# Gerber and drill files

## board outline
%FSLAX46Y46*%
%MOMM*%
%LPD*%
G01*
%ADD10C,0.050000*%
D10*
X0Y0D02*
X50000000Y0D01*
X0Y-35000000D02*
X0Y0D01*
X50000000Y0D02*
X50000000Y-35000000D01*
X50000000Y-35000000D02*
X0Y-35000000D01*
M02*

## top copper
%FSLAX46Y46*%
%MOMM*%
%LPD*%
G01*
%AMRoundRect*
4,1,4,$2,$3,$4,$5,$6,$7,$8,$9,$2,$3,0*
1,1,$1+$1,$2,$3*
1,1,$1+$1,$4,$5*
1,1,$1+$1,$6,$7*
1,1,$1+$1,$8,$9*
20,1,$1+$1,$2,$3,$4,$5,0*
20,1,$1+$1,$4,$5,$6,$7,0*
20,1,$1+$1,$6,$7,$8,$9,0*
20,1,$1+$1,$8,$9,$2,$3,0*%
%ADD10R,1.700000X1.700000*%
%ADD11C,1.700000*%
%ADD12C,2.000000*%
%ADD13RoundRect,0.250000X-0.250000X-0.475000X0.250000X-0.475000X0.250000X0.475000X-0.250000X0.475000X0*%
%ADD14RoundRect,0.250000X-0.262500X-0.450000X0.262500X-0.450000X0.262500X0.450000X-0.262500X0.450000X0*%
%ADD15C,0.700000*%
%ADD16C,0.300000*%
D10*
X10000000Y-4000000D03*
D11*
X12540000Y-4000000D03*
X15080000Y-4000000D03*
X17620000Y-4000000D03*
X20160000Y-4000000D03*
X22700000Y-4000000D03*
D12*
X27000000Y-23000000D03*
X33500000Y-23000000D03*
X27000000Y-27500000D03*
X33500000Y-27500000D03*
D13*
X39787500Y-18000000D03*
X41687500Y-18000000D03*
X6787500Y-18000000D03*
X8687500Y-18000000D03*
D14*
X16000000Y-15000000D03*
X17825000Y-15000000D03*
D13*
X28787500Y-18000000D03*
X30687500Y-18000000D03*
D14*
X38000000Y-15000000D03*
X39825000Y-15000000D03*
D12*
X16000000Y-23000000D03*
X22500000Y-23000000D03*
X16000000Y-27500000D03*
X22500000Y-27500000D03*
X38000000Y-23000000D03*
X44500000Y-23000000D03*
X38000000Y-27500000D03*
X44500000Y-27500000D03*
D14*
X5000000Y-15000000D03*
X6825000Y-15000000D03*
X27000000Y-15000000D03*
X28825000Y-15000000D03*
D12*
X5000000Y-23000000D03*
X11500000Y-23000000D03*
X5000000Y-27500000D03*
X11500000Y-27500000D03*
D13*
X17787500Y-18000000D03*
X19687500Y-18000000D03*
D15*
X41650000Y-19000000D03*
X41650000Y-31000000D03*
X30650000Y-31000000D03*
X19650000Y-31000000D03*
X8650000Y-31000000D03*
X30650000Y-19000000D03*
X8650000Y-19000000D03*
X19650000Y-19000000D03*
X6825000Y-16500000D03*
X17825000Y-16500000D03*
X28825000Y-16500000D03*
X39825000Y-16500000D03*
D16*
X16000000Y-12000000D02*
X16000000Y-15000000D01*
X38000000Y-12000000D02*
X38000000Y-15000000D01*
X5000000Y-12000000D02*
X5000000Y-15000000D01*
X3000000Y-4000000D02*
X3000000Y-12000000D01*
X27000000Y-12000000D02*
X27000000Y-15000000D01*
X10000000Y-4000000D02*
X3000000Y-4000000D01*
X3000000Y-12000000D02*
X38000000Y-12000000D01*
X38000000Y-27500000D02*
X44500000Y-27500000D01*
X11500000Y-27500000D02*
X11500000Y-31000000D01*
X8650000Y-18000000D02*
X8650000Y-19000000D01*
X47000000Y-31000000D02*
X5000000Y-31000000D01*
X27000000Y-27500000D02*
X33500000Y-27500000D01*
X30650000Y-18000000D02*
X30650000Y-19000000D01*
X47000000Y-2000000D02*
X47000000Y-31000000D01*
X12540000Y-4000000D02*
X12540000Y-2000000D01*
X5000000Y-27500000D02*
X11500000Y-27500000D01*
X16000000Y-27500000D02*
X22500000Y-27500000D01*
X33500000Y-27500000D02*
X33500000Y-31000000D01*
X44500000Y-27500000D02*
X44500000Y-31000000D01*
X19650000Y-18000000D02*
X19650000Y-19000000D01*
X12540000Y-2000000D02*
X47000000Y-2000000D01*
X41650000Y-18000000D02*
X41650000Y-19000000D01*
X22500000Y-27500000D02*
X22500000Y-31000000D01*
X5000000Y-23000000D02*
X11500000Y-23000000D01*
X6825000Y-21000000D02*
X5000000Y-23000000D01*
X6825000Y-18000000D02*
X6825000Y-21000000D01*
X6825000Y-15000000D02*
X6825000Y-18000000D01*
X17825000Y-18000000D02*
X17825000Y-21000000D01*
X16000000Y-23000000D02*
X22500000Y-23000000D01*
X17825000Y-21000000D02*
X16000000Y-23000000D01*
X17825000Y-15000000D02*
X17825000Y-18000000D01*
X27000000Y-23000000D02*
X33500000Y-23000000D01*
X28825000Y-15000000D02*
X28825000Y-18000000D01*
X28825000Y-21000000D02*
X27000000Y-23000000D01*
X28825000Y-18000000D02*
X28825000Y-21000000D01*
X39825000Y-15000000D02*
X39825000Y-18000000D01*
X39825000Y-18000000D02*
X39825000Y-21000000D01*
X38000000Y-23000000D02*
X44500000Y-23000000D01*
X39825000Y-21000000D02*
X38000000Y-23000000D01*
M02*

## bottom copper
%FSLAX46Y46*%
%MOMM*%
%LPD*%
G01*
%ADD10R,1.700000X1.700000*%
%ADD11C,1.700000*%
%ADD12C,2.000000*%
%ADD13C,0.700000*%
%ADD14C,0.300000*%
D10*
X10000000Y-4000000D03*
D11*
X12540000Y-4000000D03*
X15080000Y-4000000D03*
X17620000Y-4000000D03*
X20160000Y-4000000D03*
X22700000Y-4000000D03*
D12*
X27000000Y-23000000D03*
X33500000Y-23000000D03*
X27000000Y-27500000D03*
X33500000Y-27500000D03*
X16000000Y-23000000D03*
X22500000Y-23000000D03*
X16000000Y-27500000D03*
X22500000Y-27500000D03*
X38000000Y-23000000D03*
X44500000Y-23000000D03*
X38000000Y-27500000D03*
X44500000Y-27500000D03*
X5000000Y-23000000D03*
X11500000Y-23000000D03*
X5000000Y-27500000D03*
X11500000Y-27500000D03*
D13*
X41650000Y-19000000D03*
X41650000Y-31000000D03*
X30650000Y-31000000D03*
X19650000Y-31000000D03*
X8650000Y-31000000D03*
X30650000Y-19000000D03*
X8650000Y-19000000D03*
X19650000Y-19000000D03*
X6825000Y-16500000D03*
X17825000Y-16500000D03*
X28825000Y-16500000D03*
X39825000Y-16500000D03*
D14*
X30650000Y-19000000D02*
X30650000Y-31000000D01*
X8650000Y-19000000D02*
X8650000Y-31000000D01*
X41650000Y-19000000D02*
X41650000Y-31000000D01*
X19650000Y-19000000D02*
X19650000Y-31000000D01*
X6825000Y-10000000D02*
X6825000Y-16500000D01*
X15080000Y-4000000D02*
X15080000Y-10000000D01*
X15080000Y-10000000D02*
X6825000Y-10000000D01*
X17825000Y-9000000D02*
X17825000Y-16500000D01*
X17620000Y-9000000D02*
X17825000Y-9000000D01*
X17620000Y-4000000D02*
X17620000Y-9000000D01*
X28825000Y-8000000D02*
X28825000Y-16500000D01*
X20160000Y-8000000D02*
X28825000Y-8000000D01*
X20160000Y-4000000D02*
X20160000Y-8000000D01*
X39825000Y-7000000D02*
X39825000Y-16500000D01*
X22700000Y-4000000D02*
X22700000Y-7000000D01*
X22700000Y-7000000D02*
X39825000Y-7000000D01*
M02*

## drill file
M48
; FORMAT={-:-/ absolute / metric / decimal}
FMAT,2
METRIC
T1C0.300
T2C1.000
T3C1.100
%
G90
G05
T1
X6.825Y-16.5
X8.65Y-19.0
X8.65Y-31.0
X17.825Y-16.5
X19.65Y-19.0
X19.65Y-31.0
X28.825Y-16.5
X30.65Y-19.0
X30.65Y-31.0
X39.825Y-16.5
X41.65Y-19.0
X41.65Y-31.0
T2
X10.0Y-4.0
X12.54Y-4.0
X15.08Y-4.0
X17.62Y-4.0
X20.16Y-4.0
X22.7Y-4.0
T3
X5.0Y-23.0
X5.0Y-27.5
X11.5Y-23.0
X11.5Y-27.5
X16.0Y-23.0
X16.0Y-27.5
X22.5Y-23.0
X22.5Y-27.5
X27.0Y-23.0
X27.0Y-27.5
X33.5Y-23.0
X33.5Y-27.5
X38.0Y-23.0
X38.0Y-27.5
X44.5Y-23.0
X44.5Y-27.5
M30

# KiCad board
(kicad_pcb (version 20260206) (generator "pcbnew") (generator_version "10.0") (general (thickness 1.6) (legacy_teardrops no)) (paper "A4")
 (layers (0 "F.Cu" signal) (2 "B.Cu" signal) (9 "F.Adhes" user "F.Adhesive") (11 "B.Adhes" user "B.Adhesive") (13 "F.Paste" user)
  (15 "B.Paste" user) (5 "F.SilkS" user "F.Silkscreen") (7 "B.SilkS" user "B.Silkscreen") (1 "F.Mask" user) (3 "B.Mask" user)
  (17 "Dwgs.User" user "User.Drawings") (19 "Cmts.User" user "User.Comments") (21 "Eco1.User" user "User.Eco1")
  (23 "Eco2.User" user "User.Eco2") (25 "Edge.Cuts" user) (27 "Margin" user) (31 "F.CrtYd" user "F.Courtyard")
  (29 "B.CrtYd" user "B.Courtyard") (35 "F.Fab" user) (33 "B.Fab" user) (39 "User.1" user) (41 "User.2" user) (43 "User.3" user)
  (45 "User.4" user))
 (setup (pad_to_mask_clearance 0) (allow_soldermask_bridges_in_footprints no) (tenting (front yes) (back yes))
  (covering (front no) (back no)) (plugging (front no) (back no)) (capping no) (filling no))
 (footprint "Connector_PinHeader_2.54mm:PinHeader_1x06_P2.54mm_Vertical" (layer "F.Cu") (at 10 4 90)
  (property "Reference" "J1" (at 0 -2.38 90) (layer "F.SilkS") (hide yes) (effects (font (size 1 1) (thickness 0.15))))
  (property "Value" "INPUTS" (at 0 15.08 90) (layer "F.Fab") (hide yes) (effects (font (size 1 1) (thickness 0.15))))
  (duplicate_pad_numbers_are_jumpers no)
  (pad "1" thru_hole rect (at 0 0 90) (size 1.7 1.7) (drill 1) (layers "*.Cu" "*.Mask") (remove_unused_layers no) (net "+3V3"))
  (pad "2" thru_hole circle (at 0 2.54 90) (size 1.7 1.7) (drill 1) (layers "*.Cu" "*.Mask") (remove_unused_layers no) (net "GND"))
  (pad "3" thru_hole circle (at 0 5.08 90) (size 1.7 1.7) (drill 1) (layers "*.Cu" "*.Mask") (remove_unused_layers no) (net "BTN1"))
  (pad "4" thru_hole circle (at 0 7.62 90) (size 1.7 1.7) (drill 1) (layers "*.Cu" "*.Mask") (remove_unused_layers no) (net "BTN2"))
  (pad "5" thru_hole circle (at 0 10.16 90) (size 1.7 1.7) (drill 1) (layers "*.Cu" "*.Mask") (remove_unused_layers no) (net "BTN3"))
  (pad "6" thru_hole circle (at 0 12.7 90) (size 1.7 1.7) (drill 1) (layers "*.Cu" "*.Mask") (remove_unused_layers no) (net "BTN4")))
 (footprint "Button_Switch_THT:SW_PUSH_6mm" (layer "F.Cu") (at 27 23)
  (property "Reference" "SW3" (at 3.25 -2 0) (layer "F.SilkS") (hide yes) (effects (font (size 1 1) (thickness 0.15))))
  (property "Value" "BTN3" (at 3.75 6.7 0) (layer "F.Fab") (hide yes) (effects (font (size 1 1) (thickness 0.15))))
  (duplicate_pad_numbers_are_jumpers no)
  (pad "1" thru_hole circle (at 0 0 90) (size 2 2) (drill 1.1) (layers "*.Cu" "*.Mask") (remove_unused_layers no) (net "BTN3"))
  (pad "1" thru_hole circle (at 6.5 0 90) (size 2 2) (drill 1.1) (layers "*.Cu" "*.Mask") (remove_unused_layers no) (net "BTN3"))
  (pad "2" thru_hole circle (at 0 4.5 90) (size 2 2) (drill 1.1) (layers "*.Cu" "*.Mask") (remove_unused_layers no) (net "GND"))
  (pad "2" thru_hole circle (at 6.5 4.5 90) (size 2 2) (drill 1.1) (layers "*.Cu" "*.Mask") (remove_unused_layers no) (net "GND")))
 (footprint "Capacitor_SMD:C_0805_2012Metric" (layer "F.Cu") (at 40.7375 18)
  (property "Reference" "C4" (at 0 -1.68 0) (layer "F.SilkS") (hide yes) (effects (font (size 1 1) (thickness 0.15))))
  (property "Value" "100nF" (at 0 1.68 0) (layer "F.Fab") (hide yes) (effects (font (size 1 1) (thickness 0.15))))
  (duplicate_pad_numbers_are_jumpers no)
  (pad "1" smd roundrect (at -0.95 0) (size 1 1.45) (layers "F.Cu" "F.Mask" "F.Paste") (roundrect_rratio 0.25) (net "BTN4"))
  (pad "2" smd roundrect (at 0.95 0) (size 1 1.45) (layers "F.Cu" "F.Mask" "F.Paste") (roundrect_rratio 0.25) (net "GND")))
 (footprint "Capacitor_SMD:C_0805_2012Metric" (layer "F.Cu") (at 7.7375 18)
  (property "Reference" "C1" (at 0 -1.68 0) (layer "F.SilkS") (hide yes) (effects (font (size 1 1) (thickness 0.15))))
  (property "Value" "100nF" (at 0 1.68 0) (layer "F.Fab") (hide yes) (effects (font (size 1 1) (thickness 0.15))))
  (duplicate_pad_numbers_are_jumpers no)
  (pad "1" smd roundrect (at -0.95 0) (size 1 1.45) (layers "F.Cu" "F.Mask" "F.Paste") (roundrect_rratio 0.25) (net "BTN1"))
  (pad "2" smd roundrect (at 0.95 0) (size 1 1.45) (layers "F.Cu" "F.Mask" "F.Paste") (roundrect_rratio 0.25) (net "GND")))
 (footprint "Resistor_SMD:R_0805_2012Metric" (layer "F.Cu") (at 16.9125 15)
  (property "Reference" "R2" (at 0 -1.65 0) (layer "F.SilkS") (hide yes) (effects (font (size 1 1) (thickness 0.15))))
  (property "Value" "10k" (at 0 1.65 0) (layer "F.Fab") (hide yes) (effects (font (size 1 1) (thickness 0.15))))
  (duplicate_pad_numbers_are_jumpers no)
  (pad "1" smd roundrect (at -0.9125 0) (size 1.025 1.4) (layers "F.Cu" "F.Mask" "F.Paste") (roundrect_rratio 0.243902) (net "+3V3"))
  (pad "2" smd roundrect (at 0.9125 0) (size 1.025 1.4) (layers "F.Cu" "F.Mask" "F.Paste") (roundrect_rratio 0.243902) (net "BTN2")))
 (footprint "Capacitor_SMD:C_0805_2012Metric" (layer "F.Cu") (at 29.7375 18)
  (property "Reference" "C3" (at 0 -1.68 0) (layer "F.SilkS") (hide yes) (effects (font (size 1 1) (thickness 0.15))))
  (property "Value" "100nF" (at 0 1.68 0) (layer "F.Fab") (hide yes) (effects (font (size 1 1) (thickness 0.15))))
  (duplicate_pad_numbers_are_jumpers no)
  (pad "1" smd roundrect (at -0.95 0) (size 1 1.45) (layers "F.Cu" "F.Mask" "F.Paste") (roundrect_rratio 0.25) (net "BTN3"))
  (pad "2" smd roundrect (at 0.95 0) (size 1 1.45) (layers "F.Cu" "F.Mask" "F.Paste") (roundrect_rratio 0.25) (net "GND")))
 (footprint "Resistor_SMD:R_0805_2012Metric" (layer "F.Cu") (at 38.9125 15)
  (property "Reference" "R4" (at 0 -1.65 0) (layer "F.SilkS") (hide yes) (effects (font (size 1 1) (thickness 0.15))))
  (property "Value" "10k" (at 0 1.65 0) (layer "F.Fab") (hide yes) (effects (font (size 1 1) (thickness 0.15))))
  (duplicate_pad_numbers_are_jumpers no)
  (pad "1" smd roundrect (at -0.9125 0) (size 1.025 1.4) (layers "F.Cu" "F.Mask" "F.Paste") (roundrect_rratio 0.243902) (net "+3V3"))
  (pad "2" smd roundrect (at 0.9125 0) (size 1.025 1.4) (layers "F.Cu" "F.Mask" "F.Paste") (roundrect_rratio 0.243902) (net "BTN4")))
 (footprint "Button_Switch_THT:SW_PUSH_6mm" (layer "F.Cu") (at 16 23)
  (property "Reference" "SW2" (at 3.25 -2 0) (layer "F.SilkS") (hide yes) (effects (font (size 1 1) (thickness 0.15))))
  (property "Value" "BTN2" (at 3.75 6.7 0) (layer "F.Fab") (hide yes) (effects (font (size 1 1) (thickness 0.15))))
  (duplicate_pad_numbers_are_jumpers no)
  (pad "1" thru_hole circle (at 0 0 90) (size 2 2) (drill 1.1) (layers "*.Cu" "*.Mask") (remove_unused_layers no) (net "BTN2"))
  (pad "1" thru_hole circle (at 6.5 0 90) (size 2 2) (drill 1.1) (layers "*.Cu" "*.Mask") (remove_unused_layers no) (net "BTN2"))
  (pad "2" thru_hole circle (at 0 4.5 90) (size 2 2) (drill 1.1) (layers "*.Cu" "*.Mask") (remove_unused_layers no) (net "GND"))
  (pad "2" thru_hole circle (at 6.5 4.5 90) (size 2 2) (drill 1.1) (layers "*.Cu" "*.Mask") (remove_unused_layers no) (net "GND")))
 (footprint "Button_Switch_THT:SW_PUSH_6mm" (layer "F.Cu") (at 38 23)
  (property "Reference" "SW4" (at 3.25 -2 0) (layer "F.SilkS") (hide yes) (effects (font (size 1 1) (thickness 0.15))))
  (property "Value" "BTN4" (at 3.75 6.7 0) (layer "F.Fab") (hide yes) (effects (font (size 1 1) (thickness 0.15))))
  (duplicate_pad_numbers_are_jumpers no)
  (pad "1" thru_hole circle (at 0 0 90) (size 2 2) (drill 1.1) (layers "*.Cu" "*.Mask") (remove_unused_layers no) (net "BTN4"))
  (pad "1" thru_hole circle (at 6.5 0 90) (size 2 2) (drill 1.1) (layers "*.Cu" "*.Mask") (remove_unused_layers no) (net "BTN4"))
  (pad "2" thru_hole circle (at 0 4.5 90) (size 2 2) (drill 1.1) (layers "*.Cu" "*.Mask") (remove_unused_layers no) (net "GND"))
  (pad "2" thru_hole circle (at 6.5 4.5 90) (size 2 2) (drill 1.1) (layers "*.Cu" "*.Mask") (remove_unused_layers no) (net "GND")))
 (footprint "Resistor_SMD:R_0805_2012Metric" (layer "F.Cu") (at 5.9125 15)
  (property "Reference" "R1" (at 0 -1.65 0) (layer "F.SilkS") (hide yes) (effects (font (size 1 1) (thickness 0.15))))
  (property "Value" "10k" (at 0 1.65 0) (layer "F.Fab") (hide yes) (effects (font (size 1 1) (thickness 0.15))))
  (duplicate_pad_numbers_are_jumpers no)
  (pad "1" smd roundrect (at -0.9125 0) (size 1.025 1.4) (layers "F.Cu" "F.Mask" "F.Paste") (roundrect_rratio 0.243902) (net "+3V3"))
  (pad "2" smd roundrect (at 0.9125 0) (size 1.025 1.4) (layers "F.Cu" "F.Mask" "F.Paste") (roundrect_rratio 0.243902) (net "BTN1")))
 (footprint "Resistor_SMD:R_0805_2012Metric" (layer "F.Cu") (at 27.9125 15)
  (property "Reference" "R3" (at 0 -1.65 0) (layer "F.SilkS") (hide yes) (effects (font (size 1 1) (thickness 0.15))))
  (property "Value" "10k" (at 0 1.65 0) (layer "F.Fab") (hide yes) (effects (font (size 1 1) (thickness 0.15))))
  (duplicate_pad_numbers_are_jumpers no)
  (pad "1" smd roundrect (at -0.9125 0) (size 1.025 1.4) (layers "F.Cu" "F.Mask" "F.Paste") (roundrect_rratio 0.243902) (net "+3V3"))
  (pad "2" smd roundrect (at 0.9125 0) (size 1.025 1.4) (layers "F.Cu" "F.Mask" "F.Paste") (roundrect_rratio 0.243902) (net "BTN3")))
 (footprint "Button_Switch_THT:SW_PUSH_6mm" (layer "F.Cu") (at 5 23)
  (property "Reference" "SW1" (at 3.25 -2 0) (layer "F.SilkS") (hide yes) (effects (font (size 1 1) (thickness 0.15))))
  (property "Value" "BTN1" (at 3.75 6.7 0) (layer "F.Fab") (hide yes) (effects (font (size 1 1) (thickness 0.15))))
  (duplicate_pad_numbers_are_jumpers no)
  (pad "1" thru_hole circle (at 0 0 90) (size 2 2) (drill 1.1) (layers "*.Cu" "*.Mask") (remove_unused_layers no) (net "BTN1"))
  (pad "1" thru_hole circle (at 6.5 0 90) (size 2 2) (drill 1.1) (layers "*.Cu" "*.Mask") (remove_unused_layers no) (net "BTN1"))
  (pad "2" thru_hole circle (at 0 4.5 90) (size 2 2) (drill 1.1) (layers "*.Cu" "*.Mask") (remove_unused_layers no) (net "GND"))
  (pad "2" thru_hole circle (at 6.5 4.5 90) (size 2 2) (drill 1.1) (layers "*.Cu" "*.Mask") (remove_unused_layers no) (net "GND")))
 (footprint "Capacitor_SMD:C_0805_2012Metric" (layer "F.Cu") (at 18.7375 18)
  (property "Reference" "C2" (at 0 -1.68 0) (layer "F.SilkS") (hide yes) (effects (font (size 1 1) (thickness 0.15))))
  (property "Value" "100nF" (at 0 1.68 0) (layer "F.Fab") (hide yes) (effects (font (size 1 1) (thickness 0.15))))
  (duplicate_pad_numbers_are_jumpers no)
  (pad "1" smd roundrect (at -0.95 0) (size 1 1.45) (layers "F.Cu" "F.Mask" "F.Paste") (roundrect_rratio 0.25) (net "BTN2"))
  (pad "2" smd roundrect (at 0.95 0) (size 1 1.45) (layers "F.Cu" "F.Mask" "F.Paste") (roundrect_rratio 0.25) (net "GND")))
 (gr_line (start 0 0) (end 50 0) (stroke (width 0.05) (type default)) (layer "Edge.Cuts"))
 (gr_line (start 0 35) (end 0 0) (stroke (width 0.05) (type default)) (layer "Edge.Cuts"))
 (gr_line (start 50 0) (end 50 35) (stroke (width 0.05) (type default)) (layer "Edge.Cuts"))
 (gr_line (start 50 35) (end 0 35) (stroke (width 0.05) (type default)) (layer "Edge.Cuts"))
 (segment (start 16 12) (end 16 15) (width 0.3) (layer "F.Cu") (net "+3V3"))
 (segment (start 38 12) (end 38 15) (width 0.3) (layer "F.Cu") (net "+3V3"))
 (segment (start 5 12) (end 5 15) (width 0.3) (layer "F.Cu") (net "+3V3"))
 (segment (start 3 4) (end 3 12) (width 0.3) (layer "F.Cu") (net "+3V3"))
 (segment (start 27 12) (end 27 15) (width 0.3) (layer "F.Cu") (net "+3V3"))
 (segment (start 10 4) (end 3 4) (width 0.3) (layer "F.Cu") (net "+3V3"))
 (segment (start 3 12) (end 38 12) (width 0.3) (layer "F.Cu") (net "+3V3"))
 (segment (start 38 27.5) (end 44.5 27.5) (width 0.3) (layer "F.Cu") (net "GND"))
 (segment (start 11.5 27.5) (end 11.5 31) (width 0.3) (layer "F.Cu") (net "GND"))
 (segment (start 8.65 18) (end 8.65 19) (width 0.3) (layer "F.Cu") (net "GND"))
 (segment (start 47 31) (end 5 31) (width 0.3) (layer "F.Cu") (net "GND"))
 (segment (start 27 27.5) (end 33.5 27.5) (width 0.3) (layer "F.Cu") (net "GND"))
 (segment (start 30.65 18) (end 30.65 19) (width 0.3) (layer "F.Cu") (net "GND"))
 (segment (start 47 2) (end 47 31) (width 0.3) (layer "F.Cu") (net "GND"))
 (segment (start 12.54 4) (end 12.54 2) (width 0.3) (layer "F.Cu") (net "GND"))
 (segment (start 5 27.5) (end 11.5 27.5) (width 0.3) (layer "F.Cu") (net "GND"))
 (segment (start 16 27.5) (end 22.5 27.5) (width 0.3) (layer "F.Cu") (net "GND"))
 (segment (start 33.5 27.5) (end 33.5 31) (width 0.3) (layer "F.Cu") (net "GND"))
 (segment (start 44.5 27.5) (end 44.5 31) (width 0.3) (layer "F.Cu") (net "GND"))
 (segment (start 19.65 18) (end 19.65 19) (width 0.3) (layer "F.Cu") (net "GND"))
 (segment (start 12.54 2) (end 47 2) (width 0.3) (layer "F.Cu") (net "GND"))
 (segment (start 41.65 18) (end 41.65 19) (width 0.3) (layer "F.Cu") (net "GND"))
 (segment (start 22.5 27.5) (end 22.5 31) (width 0.3) (layer "F.Cu") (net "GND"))
 (via (at 41.65 19) (size 0.7) (drill 0.3) (layers "F.Cu" "B.Cu") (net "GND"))
 (via (at 41.65 31) (size 0.7) (drill 0.3) (layers "F.Cu" "B.Cu") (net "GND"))
 (via (at 30.65 31) (size 0.7) (drill 0.3) (layers "F.Cu" "B.Cu") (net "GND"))
 (via (at 19.65 31) (size 0.7) (drill 0.3) (layers "F.Cu" "B.Cu") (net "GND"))
 (via (at 8.65 31) (size 0.7) (drill 0.3) (layers "F.Cu" "B.Cu") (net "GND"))
 (via (at 30.65 19) (size 0.7) (drill 0.3) (layers "F.Cu" "B.Cu") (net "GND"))
 (via (at 8.65 19) (size 0.7) (drill 0.3) (layers "F.Cu" "B.Cu") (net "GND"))
 (via (at 19.65 19) (size 0.7) (drill 0.3) (layers "F.Cu" "B.Cu") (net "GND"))
 (segment (start 30.65 19) (end 30.65 31) (width 0.3) (layer "B.Cu") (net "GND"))
 (segment (start 8.65 19) (end 8.65 31) (width 0.3) (layer "B.Cu") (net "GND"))
 (segment (start 41.65 19) (end 41.65 31) (width 0.3) (layer "B.Cu") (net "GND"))
 (segment (start 19.65 19) (end 19.65 31) (width 0.3) (layer "B.Cu") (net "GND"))
 (segment (start 5 23) (end 11.5 23) (width 0.3) (layer "F.Cu") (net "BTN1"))
 (segment (start 6.825 21) (end 5 23) (width 0.3) (layer "F.Cu") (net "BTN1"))
 (segment (start 6.825 18) (end 6.825 21) (width 0.3) (layer "F.Cu") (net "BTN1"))
 (segment (start 6.825 15) (end 6.825 18) (width 0.3) (layer "F.Cu") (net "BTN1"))
 (via (at 6.825 16.5) (size 0.7) (drill 0.3) (layers "F.Cu" "B.Cu") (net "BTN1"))
 (segment (start 6.825 10) (end 6.825 16.5) (width 0.3) (layer "B.Cu") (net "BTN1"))
 (segment (start 15.08 4) (end 15.08 10) (width 0.3) (layer "B.Cu") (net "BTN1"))
 (segment (start 15.08 10) (end 6.825 10) (width 0.3) (layer "B.Cu") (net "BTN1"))
 (segment (start 17.825 18) (end 17.825 21) (width 0.3) (layer "F.Cu") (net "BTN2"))
 (segment (start 16 23) (end 22.5 23) (width 0.3) (layer "F.Cu") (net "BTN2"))
 (segment (start 17.825 21) (end 16 23) (width 0.3) (layer "F.Cu") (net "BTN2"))
 (segment (start 17.825 15) (end 17.825 18) (width 0.3) (layer "F.Cu") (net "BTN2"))
 (via (at 17.825 16.5) (size 0.7) (drill 0.3) (layers "F.Cu" "B.Cu") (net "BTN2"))
 (segment (start 17.825 9) (end 17.825 16.5) (width 0.3) (layer "B.Cu") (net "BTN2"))
 (segment (start 17.62 9) (end 17.825 9) (width 0.3) (layer "B.Cu") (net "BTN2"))
 (segment (start 17.62 4) (end 17.62 9) (width 0.3) (layer "B.Cu") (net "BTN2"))
 (segment (start 27 23) (end 33.5 23) (width 0.3) (layer "F.Cu") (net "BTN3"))
 (segment (start 28.825 15) (end 28.825 18) (width 0.3) (layer "F.Cu") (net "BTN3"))
 (segment (start 28.825 21) (end 27 23) (width 0.3) (layer "F.Cu") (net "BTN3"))
 (segment (start 28.825 18) (end 28.825 21) (width 0.3) (layer "F.Cu") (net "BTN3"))
 (via (at 28.825 16.5) (size 0.7) (drill 0.3) (layers "F.Cu" "B.Cu") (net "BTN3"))
 (segment (start 28.825 8) (end 28.825 16.5) (width 0.3) (layer "B.Cu") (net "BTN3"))
 (segment (start 20.16 8) (end 28.825 8) (width 0.3) (layer "B.Cu") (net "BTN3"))
 (segment (start 20.16 4) (end 20.16 8) (width 0.3) (layer "B.Cu") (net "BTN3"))
 (segment (start 39.825 15) (end 39.825 18) (width 0.3) (layer "F.Cu") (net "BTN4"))
 (segment (start 39.825 18) (end 39.825 21) (width 0.3) (layer "F.Cu") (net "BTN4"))
 (segment (start 38 23) (end 44.5 23) (width 0.3) (layer "F.Cu") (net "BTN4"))
 (segment (start 39.825 21) (end 38 23) (width 0.3) (layer "F.Cu") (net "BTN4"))
 (via (at 39.825 16.5) (size 0.7) (drill 0.3) (layers "F.Cu" "B.Cu") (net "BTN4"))
 (segment (start 39.825 7) (end 39.825 16.5) (width 0.3) (layer "B.Cu") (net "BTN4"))
 (segment (start 22.7 4) (end 22.7 7) (width 0.3) (layer "B.Cu") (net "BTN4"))
 (segment (start 22.7 7) (end 39.825 7) (width 0.3) (layer "B.Cu") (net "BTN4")))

